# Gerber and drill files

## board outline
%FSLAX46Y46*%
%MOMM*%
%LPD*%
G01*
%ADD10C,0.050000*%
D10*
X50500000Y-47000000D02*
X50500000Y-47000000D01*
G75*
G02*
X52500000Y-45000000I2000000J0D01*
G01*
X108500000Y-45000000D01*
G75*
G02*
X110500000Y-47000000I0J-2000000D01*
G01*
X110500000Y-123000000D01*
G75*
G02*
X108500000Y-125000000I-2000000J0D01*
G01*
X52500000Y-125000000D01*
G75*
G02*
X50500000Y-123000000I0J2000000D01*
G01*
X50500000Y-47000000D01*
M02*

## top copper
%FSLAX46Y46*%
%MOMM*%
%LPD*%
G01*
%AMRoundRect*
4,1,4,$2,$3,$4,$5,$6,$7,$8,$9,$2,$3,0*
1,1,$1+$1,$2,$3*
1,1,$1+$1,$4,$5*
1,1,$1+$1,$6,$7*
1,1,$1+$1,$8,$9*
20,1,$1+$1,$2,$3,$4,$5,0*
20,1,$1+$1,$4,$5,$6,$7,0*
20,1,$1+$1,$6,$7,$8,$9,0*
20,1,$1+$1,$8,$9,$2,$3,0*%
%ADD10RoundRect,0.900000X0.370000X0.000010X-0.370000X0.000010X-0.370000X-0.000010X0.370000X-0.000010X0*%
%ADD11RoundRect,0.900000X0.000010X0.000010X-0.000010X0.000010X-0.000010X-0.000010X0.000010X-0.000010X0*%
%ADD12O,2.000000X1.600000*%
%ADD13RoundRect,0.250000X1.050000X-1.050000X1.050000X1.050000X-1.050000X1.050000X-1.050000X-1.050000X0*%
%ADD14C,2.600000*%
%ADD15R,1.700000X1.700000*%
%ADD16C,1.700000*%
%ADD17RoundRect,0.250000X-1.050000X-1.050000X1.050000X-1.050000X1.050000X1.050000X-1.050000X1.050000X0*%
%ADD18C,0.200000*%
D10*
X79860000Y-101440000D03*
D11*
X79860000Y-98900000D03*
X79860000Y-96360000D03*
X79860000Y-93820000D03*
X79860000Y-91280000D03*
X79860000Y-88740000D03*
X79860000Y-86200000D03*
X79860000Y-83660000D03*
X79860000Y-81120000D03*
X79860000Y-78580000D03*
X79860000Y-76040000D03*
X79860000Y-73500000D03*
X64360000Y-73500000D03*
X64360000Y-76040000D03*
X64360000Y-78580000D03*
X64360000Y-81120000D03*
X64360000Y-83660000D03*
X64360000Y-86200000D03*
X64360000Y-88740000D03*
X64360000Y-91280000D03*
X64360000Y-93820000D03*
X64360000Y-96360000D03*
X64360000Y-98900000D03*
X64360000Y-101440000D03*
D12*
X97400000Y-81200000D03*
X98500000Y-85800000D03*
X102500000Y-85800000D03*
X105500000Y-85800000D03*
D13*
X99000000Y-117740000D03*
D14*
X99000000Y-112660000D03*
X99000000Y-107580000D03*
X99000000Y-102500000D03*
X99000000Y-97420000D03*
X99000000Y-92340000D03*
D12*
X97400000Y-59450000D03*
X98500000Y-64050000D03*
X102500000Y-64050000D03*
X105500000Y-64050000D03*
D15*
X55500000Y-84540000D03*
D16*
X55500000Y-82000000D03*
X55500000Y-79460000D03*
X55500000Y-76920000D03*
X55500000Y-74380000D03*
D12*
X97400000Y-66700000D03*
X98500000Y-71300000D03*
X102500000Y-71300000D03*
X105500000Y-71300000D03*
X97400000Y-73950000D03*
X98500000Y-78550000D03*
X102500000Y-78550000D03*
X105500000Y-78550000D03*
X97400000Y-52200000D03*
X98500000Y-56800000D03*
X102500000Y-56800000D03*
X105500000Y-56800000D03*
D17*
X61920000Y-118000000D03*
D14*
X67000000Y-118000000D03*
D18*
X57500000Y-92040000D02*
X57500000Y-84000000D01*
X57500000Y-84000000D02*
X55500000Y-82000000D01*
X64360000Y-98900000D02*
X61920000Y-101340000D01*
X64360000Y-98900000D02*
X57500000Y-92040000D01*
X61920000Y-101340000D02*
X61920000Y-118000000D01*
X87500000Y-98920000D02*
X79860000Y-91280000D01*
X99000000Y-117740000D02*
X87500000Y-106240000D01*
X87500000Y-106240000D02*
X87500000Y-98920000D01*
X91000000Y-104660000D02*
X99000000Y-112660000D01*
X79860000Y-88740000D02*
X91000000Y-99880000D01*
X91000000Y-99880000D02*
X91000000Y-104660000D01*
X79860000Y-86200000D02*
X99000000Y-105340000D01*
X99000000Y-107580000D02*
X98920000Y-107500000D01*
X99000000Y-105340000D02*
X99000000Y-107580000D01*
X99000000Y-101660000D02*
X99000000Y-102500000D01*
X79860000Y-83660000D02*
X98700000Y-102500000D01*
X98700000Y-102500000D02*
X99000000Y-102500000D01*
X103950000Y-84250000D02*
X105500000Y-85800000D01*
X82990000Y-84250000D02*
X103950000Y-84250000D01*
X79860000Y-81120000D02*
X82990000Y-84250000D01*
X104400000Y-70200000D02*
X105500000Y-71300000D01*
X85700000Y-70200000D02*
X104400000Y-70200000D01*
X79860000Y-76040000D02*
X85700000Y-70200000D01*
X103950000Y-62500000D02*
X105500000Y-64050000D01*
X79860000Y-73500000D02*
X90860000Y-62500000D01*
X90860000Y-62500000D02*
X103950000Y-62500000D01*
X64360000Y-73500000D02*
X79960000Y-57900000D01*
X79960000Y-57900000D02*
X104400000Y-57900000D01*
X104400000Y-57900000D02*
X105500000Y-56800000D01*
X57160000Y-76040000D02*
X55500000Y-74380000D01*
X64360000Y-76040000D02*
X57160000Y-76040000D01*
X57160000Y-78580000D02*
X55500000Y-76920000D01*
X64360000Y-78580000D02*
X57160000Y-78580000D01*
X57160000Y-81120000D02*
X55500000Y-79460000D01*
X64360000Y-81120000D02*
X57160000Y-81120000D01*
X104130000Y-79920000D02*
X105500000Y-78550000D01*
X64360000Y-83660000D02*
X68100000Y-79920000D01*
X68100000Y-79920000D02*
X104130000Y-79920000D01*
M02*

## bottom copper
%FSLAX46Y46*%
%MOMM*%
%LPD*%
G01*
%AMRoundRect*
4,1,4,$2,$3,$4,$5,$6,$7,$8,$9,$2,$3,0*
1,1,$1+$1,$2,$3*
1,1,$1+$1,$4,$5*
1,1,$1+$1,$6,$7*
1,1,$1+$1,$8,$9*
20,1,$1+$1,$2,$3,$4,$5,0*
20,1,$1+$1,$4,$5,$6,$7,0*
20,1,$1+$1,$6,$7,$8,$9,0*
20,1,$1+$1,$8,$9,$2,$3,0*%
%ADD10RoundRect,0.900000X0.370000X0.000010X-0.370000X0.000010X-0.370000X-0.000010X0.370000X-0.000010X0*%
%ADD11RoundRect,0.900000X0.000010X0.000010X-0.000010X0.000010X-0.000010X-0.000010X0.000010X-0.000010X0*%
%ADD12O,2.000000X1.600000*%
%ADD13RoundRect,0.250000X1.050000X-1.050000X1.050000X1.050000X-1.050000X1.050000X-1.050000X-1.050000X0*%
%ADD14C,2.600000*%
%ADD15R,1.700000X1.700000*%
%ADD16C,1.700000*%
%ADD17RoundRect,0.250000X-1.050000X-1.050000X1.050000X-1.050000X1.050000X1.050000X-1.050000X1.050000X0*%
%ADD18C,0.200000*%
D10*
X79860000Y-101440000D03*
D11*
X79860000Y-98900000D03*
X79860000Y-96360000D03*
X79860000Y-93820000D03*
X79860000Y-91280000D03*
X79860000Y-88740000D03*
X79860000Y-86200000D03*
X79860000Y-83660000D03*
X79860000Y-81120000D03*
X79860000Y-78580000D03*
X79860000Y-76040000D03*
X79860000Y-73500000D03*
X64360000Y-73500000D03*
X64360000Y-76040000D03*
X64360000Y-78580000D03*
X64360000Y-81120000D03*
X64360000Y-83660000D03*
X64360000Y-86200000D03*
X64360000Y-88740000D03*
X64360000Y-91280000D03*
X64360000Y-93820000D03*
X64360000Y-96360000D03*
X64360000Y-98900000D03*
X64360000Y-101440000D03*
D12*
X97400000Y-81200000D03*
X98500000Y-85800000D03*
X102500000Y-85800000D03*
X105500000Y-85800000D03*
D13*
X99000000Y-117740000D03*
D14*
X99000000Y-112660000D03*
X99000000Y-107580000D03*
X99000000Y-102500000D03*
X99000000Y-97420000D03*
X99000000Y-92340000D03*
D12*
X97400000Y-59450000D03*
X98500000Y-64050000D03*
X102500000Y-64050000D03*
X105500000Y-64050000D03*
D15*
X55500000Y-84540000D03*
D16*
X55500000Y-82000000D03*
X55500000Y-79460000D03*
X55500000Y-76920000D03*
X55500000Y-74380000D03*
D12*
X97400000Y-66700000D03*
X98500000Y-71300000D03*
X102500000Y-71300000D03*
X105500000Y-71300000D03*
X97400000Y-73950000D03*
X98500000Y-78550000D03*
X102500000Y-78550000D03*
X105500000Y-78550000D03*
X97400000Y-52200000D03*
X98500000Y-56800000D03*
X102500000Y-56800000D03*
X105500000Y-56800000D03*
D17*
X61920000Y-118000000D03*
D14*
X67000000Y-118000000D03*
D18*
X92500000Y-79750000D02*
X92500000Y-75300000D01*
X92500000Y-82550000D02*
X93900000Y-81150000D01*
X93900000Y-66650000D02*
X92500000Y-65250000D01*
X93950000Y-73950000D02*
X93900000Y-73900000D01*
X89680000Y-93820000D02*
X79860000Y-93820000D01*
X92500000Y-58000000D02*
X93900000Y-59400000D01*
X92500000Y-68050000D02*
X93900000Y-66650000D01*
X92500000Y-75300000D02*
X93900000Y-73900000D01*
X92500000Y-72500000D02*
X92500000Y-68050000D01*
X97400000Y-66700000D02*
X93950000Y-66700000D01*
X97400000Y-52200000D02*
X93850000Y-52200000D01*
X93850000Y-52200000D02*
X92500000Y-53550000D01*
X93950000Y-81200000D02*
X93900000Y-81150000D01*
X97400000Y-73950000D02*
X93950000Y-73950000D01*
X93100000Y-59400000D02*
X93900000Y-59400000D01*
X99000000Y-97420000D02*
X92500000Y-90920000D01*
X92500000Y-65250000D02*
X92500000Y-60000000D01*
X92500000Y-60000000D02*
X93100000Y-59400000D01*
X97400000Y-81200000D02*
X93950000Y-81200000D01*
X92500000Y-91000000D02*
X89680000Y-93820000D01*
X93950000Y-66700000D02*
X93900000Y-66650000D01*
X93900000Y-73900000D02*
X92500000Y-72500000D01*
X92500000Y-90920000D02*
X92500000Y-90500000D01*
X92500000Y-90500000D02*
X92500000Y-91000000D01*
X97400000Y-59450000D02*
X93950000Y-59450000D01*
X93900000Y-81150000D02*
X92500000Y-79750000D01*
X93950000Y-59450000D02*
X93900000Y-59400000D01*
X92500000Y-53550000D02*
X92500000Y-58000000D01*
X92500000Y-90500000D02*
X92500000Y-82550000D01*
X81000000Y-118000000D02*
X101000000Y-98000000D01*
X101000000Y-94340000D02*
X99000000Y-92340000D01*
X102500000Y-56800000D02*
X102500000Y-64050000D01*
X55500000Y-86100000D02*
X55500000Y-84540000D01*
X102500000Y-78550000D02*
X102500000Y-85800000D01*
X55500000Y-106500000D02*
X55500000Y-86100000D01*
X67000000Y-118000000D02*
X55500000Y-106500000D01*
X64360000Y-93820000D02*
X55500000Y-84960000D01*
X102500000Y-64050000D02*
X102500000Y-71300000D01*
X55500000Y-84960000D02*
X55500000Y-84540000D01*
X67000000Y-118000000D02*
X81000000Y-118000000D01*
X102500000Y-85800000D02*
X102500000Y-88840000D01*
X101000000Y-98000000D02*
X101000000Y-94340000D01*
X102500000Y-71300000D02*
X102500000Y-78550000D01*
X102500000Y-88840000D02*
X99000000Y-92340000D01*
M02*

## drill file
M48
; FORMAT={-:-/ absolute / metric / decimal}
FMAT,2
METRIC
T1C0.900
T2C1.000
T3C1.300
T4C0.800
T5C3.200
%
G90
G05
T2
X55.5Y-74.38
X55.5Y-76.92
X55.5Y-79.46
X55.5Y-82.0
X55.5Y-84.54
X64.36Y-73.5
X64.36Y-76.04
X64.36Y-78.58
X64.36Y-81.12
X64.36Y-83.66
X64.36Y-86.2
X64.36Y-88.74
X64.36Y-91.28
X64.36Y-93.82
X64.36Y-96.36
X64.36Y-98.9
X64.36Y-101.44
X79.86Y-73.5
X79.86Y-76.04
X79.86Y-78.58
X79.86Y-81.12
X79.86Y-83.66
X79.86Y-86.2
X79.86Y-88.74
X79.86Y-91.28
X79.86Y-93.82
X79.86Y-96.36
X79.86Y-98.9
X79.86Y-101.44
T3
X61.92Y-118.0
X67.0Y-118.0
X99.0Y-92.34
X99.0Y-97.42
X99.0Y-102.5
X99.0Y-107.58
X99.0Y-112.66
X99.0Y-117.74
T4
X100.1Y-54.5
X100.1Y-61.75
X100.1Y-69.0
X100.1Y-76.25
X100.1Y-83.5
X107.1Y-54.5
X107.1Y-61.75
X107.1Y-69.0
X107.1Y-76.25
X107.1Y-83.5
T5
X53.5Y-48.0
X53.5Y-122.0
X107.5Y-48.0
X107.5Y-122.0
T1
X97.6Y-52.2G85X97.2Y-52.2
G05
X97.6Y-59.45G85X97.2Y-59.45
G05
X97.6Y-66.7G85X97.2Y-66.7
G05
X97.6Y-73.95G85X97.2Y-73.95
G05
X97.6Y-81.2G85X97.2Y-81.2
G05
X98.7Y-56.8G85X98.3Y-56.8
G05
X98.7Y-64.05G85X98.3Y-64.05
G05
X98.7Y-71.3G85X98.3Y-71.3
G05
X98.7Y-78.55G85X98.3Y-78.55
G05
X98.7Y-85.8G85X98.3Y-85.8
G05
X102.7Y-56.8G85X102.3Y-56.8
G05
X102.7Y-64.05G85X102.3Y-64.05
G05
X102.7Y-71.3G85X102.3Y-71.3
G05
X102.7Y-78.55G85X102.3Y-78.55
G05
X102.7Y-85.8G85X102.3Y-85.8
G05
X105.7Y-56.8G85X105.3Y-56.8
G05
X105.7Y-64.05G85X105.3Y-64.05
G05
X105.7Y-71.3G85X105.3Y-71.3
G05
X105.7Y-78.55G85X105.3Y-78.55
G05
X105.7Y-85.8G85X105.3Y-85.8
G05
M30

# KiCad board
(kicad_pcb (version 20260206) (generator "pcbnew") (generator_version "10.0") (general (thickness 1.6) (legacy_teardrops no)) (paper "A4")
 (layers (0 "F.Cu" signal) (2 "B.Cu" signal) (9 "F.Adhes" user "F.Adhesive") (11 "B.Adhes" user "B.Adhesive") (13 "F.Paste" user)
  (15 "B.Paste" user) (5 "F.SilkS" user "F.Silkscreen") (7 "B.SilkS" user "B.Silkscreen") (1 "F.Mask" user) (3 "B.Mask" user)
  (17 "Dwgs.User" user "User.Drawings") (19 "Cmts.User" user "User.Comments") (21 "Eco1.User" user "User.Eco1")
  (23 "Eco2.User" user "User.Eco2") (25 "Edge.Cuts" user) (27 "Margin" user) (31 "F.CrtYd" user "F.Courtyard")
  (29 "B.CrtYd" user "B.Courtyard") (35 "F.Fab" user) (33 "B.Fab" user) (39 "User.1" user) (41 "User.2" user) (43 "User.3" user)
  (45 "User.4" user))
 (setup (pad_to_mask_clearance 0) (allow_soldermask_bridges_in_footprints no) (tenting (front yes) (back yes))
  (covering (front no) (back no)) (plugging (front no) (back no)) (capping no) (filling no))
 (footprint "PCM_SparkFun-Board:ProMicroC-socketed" (layer "F.Cu") (at 72.11 88.74 180)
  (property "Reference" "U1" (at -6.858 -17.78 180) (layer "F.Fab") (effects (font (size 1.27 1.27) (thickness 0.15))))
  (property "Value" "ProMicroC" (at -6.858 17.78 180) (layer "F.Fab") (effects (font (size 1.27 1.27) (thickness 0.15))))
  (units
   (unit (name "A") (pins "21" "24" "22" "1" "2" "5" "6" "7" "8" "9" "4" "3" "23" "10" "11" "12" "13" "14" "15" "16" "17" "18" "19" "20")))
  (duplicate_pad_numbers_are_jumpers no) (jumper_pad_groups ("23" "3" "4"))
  (pad "1" thru_hole roundrect (at -7.75 -12.7 180) (size 2.54 1.8) (drill 1) (layers "*.Cu" "*.Mask") (remove_unused_layers no)
   (roundrect_rratio 0.5) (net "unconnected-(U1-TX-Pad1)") (thermal_bridge_angle 0))
  (pad "2" thru_hole roundrect (at -7.75 -10.16 180) (size 1.8 1.8) (drill 1) (layers "*.Cu" "*.Mask") (remove_unused_layers no)
   (roundrect_rratio 0.5) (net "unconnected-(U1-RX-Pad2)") (thermal_bridge_angle 0))
  (pad "3" thru_hole roundrect (at -7.75 -7.62 180) (size 1.8 1.8) (drill 1) (layers "*.Cu" "*.Mask") (remove_unused_layers no)
   (roundrect_rratio 0.5) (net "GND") (thermal_bridge_angle 0))
  (pad "4" thru_hole roundrect (at -7.75 -5.08 180) (size 1.8 1.8) (drill 1) (layers "*.Cu" "*.Mask") (remove_unused_layers no)
   (roundrect_rratio 0.5) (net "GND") (thermal_bridge_angle 0))
  (pad "5" thru_hole roundrect (at -7.75 -2.54 180) (size 1.8 1.8) (drill 1) (layers "*.Cu" "*.Mask") (remove_unused_layers no)
   (roundrect_rratio 0.5) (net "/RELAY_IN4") (thermal_bridge_angle 0))
  (pad "6" thru_hole roundrect (at -7.75 0 180) (size 1.8 1.8) (drill 1) (layers "*.Cu" "*.Mask") (remove_unused_layers no)
   (roundrect_rratio 0.5) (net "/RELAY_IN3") (thermal_bridge_angle 0))
  (pad "7" thru_hole roundrect (at -7.75 2.54 180) (size 1.8 1.8) (drill 1) (layers "*.Cu" "*.Mask") (remove_unused_layers no)
   (roundrect_rratio 0.5) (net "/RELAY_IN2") (thermal_bridge_angle 0))
  (pad "8" thru_hole roundrect (at -7.75 5.08 180) (size 1.8 1.8) (drill 1) (layers "*.Cu" "*.Mask") (remove_unused_layers no)
   (roundrect_rratio 0.5) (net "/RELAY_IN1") (thermal_bridge_angle 0))
  (pad "9" thru_hole roundrect (at -7.75 7.62 180) (size 1.8 1.8) (drill 1) (layers "*.Cu" "*.Mask") (remove_unused_layers no)
   (roundrect_rratio 0.5) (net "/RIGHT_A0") (thermal_bridge_angle 0))
  (pad "10" thru_hole roundrect (at -7.75 10.16 180) (size 1.8 1.8) (drill 1) (layers "*.Cu" "*.Mask") (remove_unused_layers no)
   (roundrect_rratio 0.5) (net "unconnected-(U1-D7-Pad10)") (thermal_bridge_angle 0))
  (pad "11" thru_hole roundrect (at -7.75 12.7 180) (size 1.8 1.8) (drill 1) (layers "*.Cu" "*.Mask") (remove_unused_layers no)
   (roundrect_rratio 0.5) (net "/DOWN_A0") (thermal_bridge_angle 0))
  (pad "12" thru_hole roundrect (at -7.75 15.24 180) (size 1.8 1.8) (drill 1) (layers "*.Cu" "*.Mask") (remove_unused_layers no)
   (roundrect_rratio 0.5) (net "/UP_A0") (thermal_bridge_angle 0))
  (pad "13" thru_hole roundrect (at 7.75 15.24 180) (size 1.8 1.8) (drill 1) (layers "*.Cu" "*.Mask") (remove_unused_layers no)
   (roundrect_rratio 0.5) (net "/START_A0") (thermal_bridge_angle 0))
  (pad "14" thru_hole roundrect (at 7.75 12.7 180) (size 1.8 1.8) (drill 1) (layers "*.Cu" "*.Mask") (remove_unused_layers no)
   (roundrect_rratio 0.5) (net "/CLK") (thermal_bridge_angle 0))
  (pad "15" thru_hole roundrect (at 7.75 10.16 180) (size 1.8 1.8) (drill 1) (layers "*.Cu" "*.Mask") (remove_unused_layers no)
   (roundrect_rratio 0.5) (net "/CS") (thermal_bridge_angle 0))
  (pad "16" thru_hole roundrect (at 7.75 7.62 180) (size 1.8 1.8) (drill 1) (layers "*.Cu" "*.Mask") (remove_unused_layers no)
   (roundrect_rratio 0.5) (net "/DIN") (thermal_bridge_angle 0))
  (pad "17" thru_hole roundrect (at 7.75 5.08 180) (size 1.8 1.8) (drill 1) (layers "*.Cu" "*.Mask") (remove_unused_layers no)
   (roundrect_rratio 0.5) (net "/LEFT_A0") (thermal_bridge_angle 0))
  (pad "18" thru_hole roundrect (at 7.75 2.54 180) (size 1.8 1.8) (drill 1) (layers "*.Cu" "*.Mask") (remove_unused_layers no)
   (roundrect_rratio 0.5) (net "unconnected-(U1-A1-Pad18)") (thermal_bridge_angle 0))
  (pad "19" thru_hole roundrect (at 7.75 0 180) (size 1.8 1.8) (drill 1) (layers "*.Cu" "*.Mask") (remove_unused_layers no)
   (roundrect_rratio 0.5) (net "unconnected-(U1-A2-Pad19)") (thermal_bridge_angle 0))
  (pad "20" thru_hole roundrect (at 7.75 -2.54 180) (size 1.8 1.8) (drill 1) (layers "*.Cu" "*.Mask") (remove_unused_layers no)
   (roundrect_rratio 0.5) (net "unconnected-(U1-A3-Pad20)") (thermal_bridge_angle 0))
  (pad "21" thru_hole roundrect (at 7.75 -5.08 180) (size 1.8 1.8) (drill 1) (layers "*.Cu" "*.Mask") (remove_unused_layers no)
   (roundrect_rratio 0.5) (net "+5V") (thermal_bridge_angle 0))
  (pad "22" thru_hole roundrect (at 7.75 -7.62 180) (size 1.8 1.8) (drill 1) (layers "*.Cu" "*.Mask") (remove_unused_layers no)
   (roundrect_rratio 0.5) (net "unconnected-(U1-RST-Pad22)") (thermal_bridge_angle 0))
  (pad "23" thru_hole roundrect (at 7.75 -10.16 180) (size 1.8 1.8) (drill 1) (layers "*.Cu" "*.Mask") (remove_unused_layers no)
   (roundrect_rratio 0.5) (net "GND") (thermal_bridge_angle 0))
  (pad "24" thru_hole roundrect (at 7.75 -12.7 180) (size 1.8 1.8) (drill 1) (layers "*.Cu" "*.Mask") (remove_unused_layers no)
   (roundrect_rratio 0.5) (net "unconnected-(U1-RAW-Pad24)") (thermal_bridge_angle 0)))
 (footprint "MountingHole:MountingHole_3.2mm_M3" (layer "F.Cu") (at 53.5 48)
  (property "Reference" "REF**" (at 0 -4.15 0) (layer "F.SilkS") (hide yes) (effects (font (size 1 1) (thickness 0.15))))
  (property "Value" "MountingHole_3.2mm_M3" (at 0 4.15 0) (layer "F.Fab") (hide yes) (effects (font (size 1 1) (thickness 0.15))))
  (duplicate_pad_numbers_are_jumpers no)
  (pad "" np_thru_hole circle (at 0 0) (size 3.2 3.2) (drill 3.2) (layers "*.Cu" "*.Mask")))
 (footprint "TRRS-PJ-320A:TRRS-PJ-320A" (layer "F.Cu") (at 108.7 83.5 -90)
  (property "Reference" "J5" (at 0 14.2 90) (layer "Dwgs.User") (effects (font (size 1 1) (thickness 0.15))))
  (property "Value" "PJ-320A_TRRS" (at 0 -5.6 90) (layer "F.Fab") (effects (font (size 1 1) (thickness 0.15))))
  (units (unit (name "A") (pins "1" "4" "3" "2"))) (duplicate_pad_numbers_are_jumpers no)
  (pad "" np_thru_hole circle (at 0 1.6 270) (size 0.8 0.8) (drill 0.8) (layers "*.Cu" "*.Mask"))
  (pad "" np_thru_hole circle (at 0 8.6 270) (size 0.8 0.8) (drill 0.8) (layers "*.Cu" "*.Mask"))
  (pad "1" thru_hole oval (at -2.3 11.3 270) (size 1.6 2) (drill oval 0.9 1.3) (layers "*.Cu" "*.Mask") (remove_unused_layers no)
   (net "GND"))
  (pad "2" thru_hole oval (at 2.3 10.2 270) (size 1.6 2) (drill oval 0.9 1.3) (layers "*.Cu" "*.Mask") (remove_unused_layers no)
   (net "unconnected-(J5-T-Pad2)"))
  (pad "3" thru_hole oval (at 2.3 6.2 270) (size 1.6 2) (drill oval 0.9 1.3) (layers "*.Cu" "*.Mask") (remove_unused_layers no) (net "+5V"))
  (pad "4" thru_hole oval (at 2.3 3.2 270) (size 1.6 2) (drill oval 0.9 1.3) (layers "*.Cu" "*.Mask") (remove_unused_layers no)
   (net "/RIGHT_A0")))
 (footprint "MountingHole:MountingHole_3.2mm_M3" (layer "F.Cu") (at 107.5 122)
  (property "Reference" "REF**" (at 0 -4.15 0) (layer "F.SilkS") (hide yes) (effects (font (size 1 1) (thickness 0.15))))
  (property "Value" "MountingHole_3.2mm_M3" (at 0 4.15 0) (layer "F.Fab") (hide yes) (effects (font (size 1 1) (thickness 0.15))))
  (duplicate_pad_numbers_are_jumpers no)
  (pad "" np_thru_hole circle (at 0 0) (size 3.2 3.2) (drill 3.2) (layers "*.Cu" "*.Mask")))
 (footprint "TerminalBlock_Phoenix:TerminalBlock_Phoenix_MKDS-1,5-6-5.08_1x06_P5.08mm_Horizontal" (layer "F.Cu") (at 99 117.74 90)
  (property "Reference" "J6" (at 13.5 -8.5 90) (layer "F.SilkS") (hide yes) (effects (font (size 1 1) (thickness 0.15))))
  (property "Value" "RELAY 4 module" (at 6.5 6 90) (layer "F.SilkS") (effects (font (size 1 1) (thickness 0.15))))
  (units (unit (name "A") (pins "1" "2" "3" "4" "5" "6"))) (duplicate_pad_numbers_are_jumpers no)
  (pad "1" thru_hole roundrect (at 0 0 90) (size 2.6 2.6) (drill 1.3) (layers "*.Cu" "*.Mask") (remove_unused_layers no)
   (roundrect_rratio 0.096154) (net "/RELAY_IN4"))
  (pad "2" thru_hole circle (at 5.08 0 90) (size 2.6 2.6) (drill 1.3) (layers "*.Cu" "*.Mask") (remove_unused_layers no) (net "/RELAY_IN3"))
  (pad "3" thru_hole circle (at 10.16 0 90) (size 2.6 2.6) (drill 1.3) (layers "*.Cu" "*.Mask") (remove_unused_layers no) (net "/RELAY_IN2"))
  (pad "4" thru_hole circle (at 15.24 0 90) (size 2.6 2.6) (drill 1.3) (layers "*.Cu" "*.Mask") (remove_unused_layers no) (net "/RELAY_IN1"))
  (pad "5" thru_hole circle (at 20.32 0 90) (size 2.6 2.6) (drill 1.3) (layers "*.Cu" "*.Mask") (remove_unused_layers no) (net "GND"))
  (pad "6" thru_hole circle (at 25.4 0 90) (size 2.6 2.6) (drill 1.3) (layers "*.Cu" "*.Mask") (remove_unused_layers no) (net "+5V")))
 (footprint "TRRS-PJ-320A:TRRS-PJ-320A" (layer "F.Cu") (at 108.7 61.75 -90)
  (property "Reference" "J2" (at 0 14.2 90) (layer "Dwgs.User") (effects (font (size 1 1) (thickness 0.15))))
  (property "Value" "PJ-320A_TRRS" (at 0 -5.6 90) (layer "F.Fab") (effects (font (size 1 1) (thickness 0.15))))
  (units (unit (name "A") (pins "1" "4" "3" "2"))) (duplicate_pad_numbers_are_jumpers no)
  (pad "" np_thru_hole circle (at 0 1.6 270) (size 0.8 0.8) (drill 0.8) (layers "*.Cu" "*.Mask"))
  (pad "" np_thru_hole circle (at 0 8.6 270) (size 0.8 0.8) (drill 0.8) (layers "*.Cu" "*.Mask"))
  (pad "1" thru_hole oval (at -2.3 11.3 270) (size 1.6 2) (drill oval 0.9 1.3) (layers "*.Cu" "*.Mask") (remove_unused_layers no)
   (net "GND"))
  (pad "2" thru_hole oval (at 2.3 10.2 270) (size 1.6 2) (drill oval 0.9 1.3) (layers "*.Cu" "*.Mask") (remove_unused_layers no)
   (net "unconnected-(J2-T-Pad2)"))
  (pad "3" thru_hole oval (at 2.3 6.2 270) (size 1.6 2) (drill oval 0.9 1.3) (layers "*.Cu" "*.Mask") (remove_unused_layers no) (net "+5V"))
  (pad "4" thru_hole oval (at 2.3 3.2 270) (size 1.6 2) (drill oval 0.9 1.3) (layers "*.Cu" "*.Mask") (remove_unused_layers no)
   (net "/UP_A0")))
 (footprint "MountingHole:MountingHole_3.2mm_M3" (layer "F.Cu") (at 107.5 48)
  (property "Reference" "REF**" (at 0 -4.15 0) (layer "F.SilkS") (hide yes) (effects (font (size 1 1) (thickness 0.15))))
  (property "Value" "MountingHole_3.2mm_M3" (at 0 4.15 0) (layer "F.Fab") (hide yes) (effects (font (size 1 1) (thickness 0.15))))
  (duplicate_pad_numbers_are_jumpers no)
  (pad "" np_thru_hole circle (at 0 0) (size 3.2 3.2) (drill 3.2) (layers "*.Cu" "*.Mask")))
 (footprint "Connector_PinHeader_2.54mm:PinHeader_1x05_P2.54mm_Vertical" (layer "F.Cu") (at 55.5 84.54 180)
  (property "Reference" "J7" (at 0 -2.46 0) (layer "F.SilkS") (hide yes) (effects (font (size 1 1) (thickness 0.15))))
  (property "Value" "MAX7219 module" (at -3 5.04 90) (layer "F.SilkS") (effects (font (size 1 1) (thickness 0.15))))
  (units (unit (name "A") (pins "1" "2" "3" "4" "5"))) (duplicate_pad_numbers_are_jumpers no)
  (pad "1" thru_hole rect (at 0 0 180) (size 1.7 1.7) (drill 1) (layers "*.Cu" "*.Mask") (remove_unused_layers no) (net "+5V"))
  (pad "2" thru_hole circle (at 0 2.54 180) (size 1.7 1.7) (drill 1) (layers "*.Cu" "*.Mask") (remove_unused_layers no) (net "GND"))
  (pad "3" thru_hole circle (at 0 5.08 180) (size 1.7 1.7) (drill 1) (layers "*.Cu" "*.Mask") (remove_unused_layers no) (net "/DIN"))
  (pad "4" thru_hole circle (at 0 7.62 180) (size 1.7 1.7) (drill 1) (layers "*.Cu" "*.Mask") (remove_unused_layers no) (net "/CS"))
  (pad "5" thru_hole circle (at 0 10.16 180) (size 1.7 1.7) (drill 1) (layers "*.Cu" "*.Mask") (remove_unused_layers no) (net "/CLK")))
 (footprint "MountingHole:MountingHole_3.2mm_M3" (layer "F.Cu") (at 53.5 122)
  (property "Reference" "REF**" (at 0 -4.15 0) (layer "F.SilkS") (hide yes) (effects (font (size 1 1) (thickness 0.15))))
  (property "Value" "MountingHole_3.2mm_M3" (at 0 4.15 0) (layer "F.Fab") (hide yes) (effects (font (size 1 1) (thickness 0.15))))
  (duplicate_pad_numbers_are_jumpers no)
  (pad "" np_thru_hole circle (at 0 0) (size 3.2 3.2) (drill 3.2) (layers "*.Cu" "*.Mask")))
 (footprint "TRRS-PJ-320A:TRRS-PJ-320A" (layer "F.Cu") (at 108.7 69 -90)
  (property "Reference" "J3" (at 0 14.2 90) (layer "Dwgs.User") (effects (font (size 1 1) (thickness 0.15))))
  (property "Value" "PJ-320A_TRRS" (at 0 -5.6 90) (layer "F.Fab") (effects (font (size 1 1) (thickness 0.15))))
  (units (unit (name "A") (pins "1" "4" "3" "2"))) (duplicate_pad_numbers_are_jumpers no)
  (pad "" np_thru_hole circle (at 0 1.6 270) (size 0.8 0.8) (drill 0.8) (layers "*.Cu" "*.Mask"))
  (pad "" np_thru_hole circle (at 0 8.6 270) (size 0.8 0.8) (drill 0.8) (layers "*.Cu" "*.Mask"))
  (pad "1" thru_hole oval (at -2.3 11.3 270) (size 1.6 2) (drill oval 0.9 1.3) (layers "*.Cu" "*.Mask") (remove_unused_layers no)
   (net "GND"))
  (pad "2" thru_hole oval (at 2.3 10.2 270) (size 1.6 2) (drill oval 0.9 1.3) (layers "*.Cu" "*.Mask") (remove_unused_layers no)
   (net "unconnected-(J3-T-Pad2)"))
  (pad "3" thru_hole oval (at 2.3 6.2 270) (size 1.6 2) (drill oval 0.9 1.3) (layers "*.Cu" "*.Mask") (remove_unused_layers no) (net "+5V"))
  (pad "4" thru_hole oval (at 2.3 3.2 270) (size 1.6 2) (drill oval 0.9 1.3) (layers "*.Cu" "*.Mask") (remove_unused_layers no)
   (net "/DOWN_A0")))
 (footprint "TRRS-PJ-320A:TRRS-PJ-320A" (layer "F.Cu") (at 108.7 76.25 -90)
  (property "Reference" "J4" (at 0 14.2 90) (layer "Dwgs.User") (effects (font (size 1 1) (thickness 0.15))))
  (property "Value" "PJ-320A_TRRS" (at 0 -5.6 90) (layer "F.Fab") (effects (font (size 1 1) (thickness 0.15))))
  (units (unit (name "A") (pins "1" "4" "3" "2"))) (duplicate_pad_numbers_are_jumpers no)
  (pad "" np_thru_hole circle (at 0 1.6 270) (size 0.8 0.8) (drill 0.8) (layers "*.Cu" "*.Mask"))
  (pad "" np_thru_hole circle (at 0 8.6 270) (size 0.8 0.8) (drill 0.8) (layers "*.Cu" "*.Mask"))
  (pad "1" thru_hole oval (at -2.3 11.3 270) (size 1.6 2) (drill oval 0.9 1.3) (layers "*.Cu" "*.Mask") (remove_unused_layers no)
   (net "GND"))
  (pad "2" thru_hole oval (at 2.3 10.2 270) (size 1.6 2) (drill oval 0.9 1.3) (layers "*.Cu" "*.Mask") (remove_unused_layers no)
   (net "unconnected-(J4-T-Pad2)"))
  (pad "3" thru_hole oval (at 2.3 6.2 270) (size 1.6 2) (drill oval 0.9 1.3) (layers "*.Cu" "*.Mask") (remove_unused_layers no) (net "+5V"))
  (pad "4" thru_hole oval (at 2.3 3.2 270) (size 1.6 2) (drill oval 0.9 1.3) (layers "*.Cu" "*.Mask") (remove_unused_layers no)
   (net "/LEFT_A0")))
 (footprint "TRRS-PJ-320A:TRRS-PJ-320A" (layer "F.Cu") (at 108.7 54.5 -90)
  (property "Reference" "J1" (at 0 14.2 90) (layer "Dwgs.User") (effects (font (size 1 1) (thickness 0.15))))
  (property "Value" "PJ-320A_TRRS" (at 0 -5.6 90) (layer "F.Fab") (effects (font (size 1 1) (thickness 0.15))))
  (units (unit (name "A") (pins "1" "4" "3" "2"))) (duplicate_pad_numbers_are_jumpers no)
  (pad "" np_thru_hole circle (at 0 1.6 270) (size 0.8 0.8) (drill 0.8) (layers "*.Cu" "*.Mask"))
  (pad "" np_thru_hole circle (at 0 8.6 270) (size 0.8 0.8) (drill 0.8) (layers "*.Cu" "*.Mask"))
  (pad "1" thru_hole oval (at -2.3 11.3 270) (size 1.6 2) (drill oval 0.9 1.3) (layers "*.Cu" "*.Mask") (remove_unused_layers no)
   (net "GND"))
  (pad "2" thru_hole oval (at 2.3 10.2 270) (size 1.6 2) (drill oval 0.9 1.3) (layers "*.Cu" "*.Mask") (remove_unused_layers no)
   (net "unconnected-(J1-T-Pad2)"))
  (pad "3" thru_hole oval (at 2.3 6.2 270) (size 1.6 2) (drill oval 0.9 1.3) (layers "*.Cu" "*.Mask") (remove_unused_layers no) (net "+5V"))
  (pad "4" thru_hole oval (at 2.3 3.2 270) (size 1.6 2) (drill oval 0.9 1.3) (layers "*.Cu" "*.Mask") (remove_unused_layers no)
   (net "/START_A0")))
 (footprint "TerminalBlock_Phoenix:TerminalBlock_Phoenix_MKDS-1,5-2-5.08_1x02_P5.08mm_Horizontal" (layer "F.Cu") (at 61.92 118)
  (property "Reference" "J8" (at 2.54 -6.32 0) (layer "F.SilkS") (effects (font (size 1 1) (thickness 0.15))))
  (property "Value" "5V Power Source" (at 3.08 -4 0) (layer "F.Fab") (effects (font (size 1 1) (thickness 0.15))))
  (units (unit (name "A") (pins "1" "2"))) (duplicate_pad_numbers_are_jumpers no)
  (pad "1" thru_hole roundrect (at 0 0) (size 2.6 2.6) (drill 1.3) (layers "*.Cu" "*.Mask") (remove_unused_layers no)
   (roundrect_rratio 0.096154) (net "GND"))
  (pad "2" thru_hole circle (at 5.08 0) (size 2.6 2.6) (drill 1.3) (layers "*.Cu" "*.Mask") (remove_unused_layers no) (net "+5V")))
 (gr_rect (start 50.5 45) (end 110.5 125) (radius 2) (stroke (width 0.05) (type solid)) (fill no) (layer "Edge.Cuts"))
 (segment (start 57.5 92.04) (end 57.5 84) (width 0.2) (layer "F.Cu") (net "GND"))
 (segment (start 57.5 84) (end 55.5 82) (width 0.2) (layer "F.Cu") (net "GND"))
 (segment (start 64.36 98.9) (end 61.92 101.34) (width 0.2) (layer "F.Cu") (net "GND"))
 (segment (start 64.36 98.9) (end 57.5 92.04) (width 0.2) (layer "F.Cu") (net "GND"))
 (segment (start 61.92 101.34) (end 61.92 118) (width 0.2) (layer "F.Cu") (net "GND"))
 (segment (start 92.5 79.75) (end 92.5 75.3) (width 0.2) (layer "B.Cu") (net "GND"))
 (segment (start 92.5 82.55) (end 93.9 81.15) (width 0.2) (layer "B.Cu") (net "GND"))
 (segment (start 93.9 66.65) (end 92.5 65.25) (width 0.2) (layer "B.Cu") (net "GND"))
 (segment (start 93.95 73.95) (end 93.9 73.9) (width 0.2) (layer "B.Cu") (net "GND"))
 (segment (start 89.68 93.82) (end 79.86 93.82) (width 0.2) (layer "B.Cu") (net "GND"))
 (segment (start 92.5 58) (end 93.9 59.4) (width 0.2) (layer "B.Cu") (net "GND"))
 (segment (start 92.5 68.05) (end 93.9 66.65) (width 0.2) (layer "B.Cu") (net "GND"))
 (segment (start 92.5 75.3) (end 93.9 73.9) (width 0.2) (layer "B.Cu") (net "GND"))
 (segment (start 92.5 72.5) (end 92.5 68.05) (width 0.2) (layer "B.Cu") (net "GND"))
 (segment (start 97.4 66.7) (end 93.95 66.7) (width 0.2) (layer "B.Cu") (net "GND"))
 (segment (start 97.4 52.2) (end 93.85 52.2) (width 0.2) (layer "B.Cu") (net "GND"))
 (segment (start 93.85 52.2) (end 92.5 53.55) (width 0.2) (layer "B.Cu") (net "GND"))
 (segment (start 93.95 81.2) (end 93.9 81.15) (width 0.2) (layer "B.Cu") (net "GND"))
 (segment (start 97.4 73.95) (end 93.95 73.95) (width 0.2) (layer "B.Cu") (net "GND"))
 (segment (start 93.1 59.4) (end 93.9 59.4) (width 0.2) (layer "B.Cu") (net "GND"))
 (segment (start 99 97.42) (end 92.5 90.92) (width 0.2) (layer "B.Cu") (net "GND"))
 (segment (start 92.5 65.25) (end 92.5 60) (width 0.2) (layer "B.Cu") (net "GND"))
 (segment (start 92.5 60) (end 93.1 59.4) (width 0.2) (layer "B.Cu") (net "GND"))
 (segment (start 97.4 81.2) (end 93.95 81.2) (width 0.2) (layer "B.Cu") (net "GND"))
 (segment (start 92.5 91) (end 89.68 93.82) (width 0.2) (layer "B.Cu") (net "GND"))
 (segment (start 93.95 66.7) (end 93.9 66.65) (width 0.2) (layer "B.Cu") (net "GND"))
 (segment (start 93.9 73.9) (end 92.5 72.5) (width 0.2) (layer "B.Cu") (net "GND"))
 (segment (start 92.5 90.92) (end 92.5 90.5) (width 0.2) (layer "B.Cu") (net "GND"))
 (segment (start 92.5 90.5) (end 92.5 91) (width 0.2) (layer "B.Cu") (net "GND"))
 (segment (start 97.4 59.45) (end 93.95 59.45) (width 0.2) (layer "B.Cu") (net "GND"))
 (segment (start 93.9 81.15) (end 92.5 79.75) (width 0.2) (layer "B.Cu") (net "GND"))
 (segment (start 93.95 59.45) (end 93.9 59.4) (width 0.2) (layer "B.Cu") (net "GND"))
 (segment (start 92.5 53.55) (end 92.5 58) (width 0.2) (layer "B.Cu") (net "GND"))
 (segment (start 92.5 90.5) (end 92.5 82.55) (width 0.2) (layer "B.Cu") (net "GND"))
 (segment (start 87.5 98.92) (end 79.86 91.28) (width 0.2) (layer "F.Cu") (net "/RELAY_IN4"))
 (segment (start 99 117.74) (end 87.5 106.24) (width 0.2) (layer "F.Cu") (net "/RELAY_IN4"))
 (segment (start 87.5 106.24) (end 87.5 98.92) (width 0.2) (layer "F.Cu") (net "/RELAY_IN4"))
 (segment (start 91 104.66) (end 99 112.66) (width 0.2) (layer "F.Cu") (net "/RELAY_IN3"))
 (segment (start 79.86 88.74) (end 91 99.88) (width 0.2) (layer "F.Cu") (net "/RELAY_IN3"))
 (segment (start 91 99.88) (end 91 104.66) (width 0.2) (layer "F.Cu") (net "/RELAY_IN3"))
 (segment (start 79.86 86.2) (end 99 105.34) (width 0.2) (layer "F.Cu") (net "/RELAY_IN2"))
 (segment (start 99 107.58) (end 98.92 107.5) (width 0.2) (layer "F.Cu") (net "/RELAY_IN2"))
 (segment (start 99 105.34) (end 99 107.58) (width 0.2) (layer "F.Cu") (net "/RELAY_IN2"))
 (segment (start 99 101.66) (end 99 102.5) (width 0.2) (layer "F.Cu") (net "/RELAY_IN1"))
 (segment (start 79.86 83.66) (end 98.7 102.5) (width 0.2) (layer "F.Cu") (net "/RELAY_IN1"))
 (segment (start 98.7 102.5) (end 99 102.5) (width 0.2) (layer "F.Cu") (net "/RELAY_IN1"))
 (segment (start 103.95 84.25) (end 105.5 85.8) (width 0.2) (layer "F.Cu") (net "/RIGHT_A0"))
 (segment (start 82.99 84.25) (end 103.95 84.25) (width 0.2) (layer "F.Cu") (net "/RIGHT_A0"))
 (segment (start 79.86 81.12) (end 82.99 84.25) (width 0.2) (layer "F.Cu") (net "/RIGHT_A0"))
 (segment (start 104.4 70.2) (end 105.5 71.3) (width 0.2) (layer "F.Cu") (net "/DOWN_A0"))
 (segment (start 85.7 70.2) (end 104.4 70.2) (width 0.2) (layer "F.Cu") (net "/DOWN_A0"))
 (segment (start 79.86 76.04) (end 85.7 70.2) (width 0.2) (layer "F.Cu") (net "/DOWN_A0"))
 (segment (start 103.95 62.5) (end 105.5 64.05) (width 0.2) (layer "F.Cu") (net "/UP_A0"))
 (segment (start 79.86 73.5) (end 90.86 62.5) (width 0.2) (layer "F.Cu") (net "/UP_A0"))
 (segment (start 90.86 62.5) (end 103.95 62.5) (width 0.2) (layer "F.Cu") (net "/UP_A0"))
 (segment (start 64.36 73.5) (end 79.96 57.9) (width 0.2) (layer "F.Cu") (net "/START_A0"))
 (segment (start 79.96 57.9) (end 104.4 57.9) (width 0.2) (layer "F.Cu") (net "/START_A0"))
 (segment (start 104.4 57.9) (end 105.5 56.8) (width 0.2) (layer "F.Cu") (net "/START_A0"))
 (segment (start 57.16 76.04) (end 55.5 74.38) (width 0.2) (layer "F.Cu") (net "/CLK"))
 (segment (start 64.36 76.04) (end 57.16 76.04) (width 0.2) (layer "F.Cu") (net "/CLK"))
 (segment (start 57.16 78.58) (end 55.5 76.92) (width 0.2) (layer "F.Cu") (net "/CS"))
 (segment (start 64.36 78.58) (end 57.16 78.58) (width 0.2) (layer "F.Cu") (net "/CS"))
 (segment (start 57.16 81.12) (end 55.5 79.46) (width 0.2) (layer "F.Cu") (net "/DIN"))
 (segment (start 64.36 81.12) (end 57.16 81.12) (width 0.2) (layer "F.Cu") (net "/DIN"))
 (segment (start 104.13 79.92) (end 105.5 78.55) (width 0.2) (layer "F.Cu") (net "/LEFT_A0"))
 (segment (start 64.36 83.66) (end 68.1 79.92) (width 0.2) (layer "F.Cu") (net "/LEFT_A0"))
 (segment (start 68.1 79.92) (end 104.13 79.92) (width 0.2) (layer "F.Cu") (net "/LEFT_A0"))
 (segment (start 81 118) (end 101 98) (width 0.2) (layer "B.Cu") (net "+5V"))
 (segment (start 101 94.34) (end 99 92.34) (width 0.2) (layer "B.Cu") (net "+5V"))
 (segment (start 102.5 56.8) (end 102.5 64.05) (width 0.2) (layer "B.Cu") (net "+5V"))
 (segment (start 55.5 86.1) (end 55.5 84.54) (width 0.2) (layer "B.Cu") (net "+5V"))
 (segment (start 102.5 78.55) (end 102.5 85.8) (width 0.2) (layer "B.Cu") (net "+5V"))
 (segment (start 55.5 106.5) (end 55.5 86.1) (width 0.2) (layer "B.Cu") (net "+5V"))
 (segment (start 67 118) (end 55.5 106.5) (width 0.2) (layer "B.Cu") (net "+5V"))
 (segment (start 64.36 93.82) (end 55.5 84.96) (width 0.2) (layer "B.Cu") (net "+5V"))
 (segment (start 102.5 64.05) (end 102.5 71.3) (width 0.2) (layer "B.Cu") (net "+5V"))
 (segment (start 55.5 84.96) (end 55.5 84.54) (width 0.2) (layer "B.Cu") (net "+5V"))
 (segment (start 67 118) (end 81 118) (width 0.2) (layer "B.Cu") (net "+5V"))
 (segment (start 102.5 85.8) (end 102.5 88.84) (width 0.2) (layer "B.Cu") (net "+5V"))
 (segment (start 101 98) (end 101 94.34) (width 0.2) (layer "B.Cu") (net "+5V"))
 (segment (start 102.5 71.3) (end 102.5 78.55) (width 0.2) (layer "B.Cu") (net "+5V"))
 (segment (start 102.5 88.84) (end 99 92.34) (width 0.2) (layer "B.Cu") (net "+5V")))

